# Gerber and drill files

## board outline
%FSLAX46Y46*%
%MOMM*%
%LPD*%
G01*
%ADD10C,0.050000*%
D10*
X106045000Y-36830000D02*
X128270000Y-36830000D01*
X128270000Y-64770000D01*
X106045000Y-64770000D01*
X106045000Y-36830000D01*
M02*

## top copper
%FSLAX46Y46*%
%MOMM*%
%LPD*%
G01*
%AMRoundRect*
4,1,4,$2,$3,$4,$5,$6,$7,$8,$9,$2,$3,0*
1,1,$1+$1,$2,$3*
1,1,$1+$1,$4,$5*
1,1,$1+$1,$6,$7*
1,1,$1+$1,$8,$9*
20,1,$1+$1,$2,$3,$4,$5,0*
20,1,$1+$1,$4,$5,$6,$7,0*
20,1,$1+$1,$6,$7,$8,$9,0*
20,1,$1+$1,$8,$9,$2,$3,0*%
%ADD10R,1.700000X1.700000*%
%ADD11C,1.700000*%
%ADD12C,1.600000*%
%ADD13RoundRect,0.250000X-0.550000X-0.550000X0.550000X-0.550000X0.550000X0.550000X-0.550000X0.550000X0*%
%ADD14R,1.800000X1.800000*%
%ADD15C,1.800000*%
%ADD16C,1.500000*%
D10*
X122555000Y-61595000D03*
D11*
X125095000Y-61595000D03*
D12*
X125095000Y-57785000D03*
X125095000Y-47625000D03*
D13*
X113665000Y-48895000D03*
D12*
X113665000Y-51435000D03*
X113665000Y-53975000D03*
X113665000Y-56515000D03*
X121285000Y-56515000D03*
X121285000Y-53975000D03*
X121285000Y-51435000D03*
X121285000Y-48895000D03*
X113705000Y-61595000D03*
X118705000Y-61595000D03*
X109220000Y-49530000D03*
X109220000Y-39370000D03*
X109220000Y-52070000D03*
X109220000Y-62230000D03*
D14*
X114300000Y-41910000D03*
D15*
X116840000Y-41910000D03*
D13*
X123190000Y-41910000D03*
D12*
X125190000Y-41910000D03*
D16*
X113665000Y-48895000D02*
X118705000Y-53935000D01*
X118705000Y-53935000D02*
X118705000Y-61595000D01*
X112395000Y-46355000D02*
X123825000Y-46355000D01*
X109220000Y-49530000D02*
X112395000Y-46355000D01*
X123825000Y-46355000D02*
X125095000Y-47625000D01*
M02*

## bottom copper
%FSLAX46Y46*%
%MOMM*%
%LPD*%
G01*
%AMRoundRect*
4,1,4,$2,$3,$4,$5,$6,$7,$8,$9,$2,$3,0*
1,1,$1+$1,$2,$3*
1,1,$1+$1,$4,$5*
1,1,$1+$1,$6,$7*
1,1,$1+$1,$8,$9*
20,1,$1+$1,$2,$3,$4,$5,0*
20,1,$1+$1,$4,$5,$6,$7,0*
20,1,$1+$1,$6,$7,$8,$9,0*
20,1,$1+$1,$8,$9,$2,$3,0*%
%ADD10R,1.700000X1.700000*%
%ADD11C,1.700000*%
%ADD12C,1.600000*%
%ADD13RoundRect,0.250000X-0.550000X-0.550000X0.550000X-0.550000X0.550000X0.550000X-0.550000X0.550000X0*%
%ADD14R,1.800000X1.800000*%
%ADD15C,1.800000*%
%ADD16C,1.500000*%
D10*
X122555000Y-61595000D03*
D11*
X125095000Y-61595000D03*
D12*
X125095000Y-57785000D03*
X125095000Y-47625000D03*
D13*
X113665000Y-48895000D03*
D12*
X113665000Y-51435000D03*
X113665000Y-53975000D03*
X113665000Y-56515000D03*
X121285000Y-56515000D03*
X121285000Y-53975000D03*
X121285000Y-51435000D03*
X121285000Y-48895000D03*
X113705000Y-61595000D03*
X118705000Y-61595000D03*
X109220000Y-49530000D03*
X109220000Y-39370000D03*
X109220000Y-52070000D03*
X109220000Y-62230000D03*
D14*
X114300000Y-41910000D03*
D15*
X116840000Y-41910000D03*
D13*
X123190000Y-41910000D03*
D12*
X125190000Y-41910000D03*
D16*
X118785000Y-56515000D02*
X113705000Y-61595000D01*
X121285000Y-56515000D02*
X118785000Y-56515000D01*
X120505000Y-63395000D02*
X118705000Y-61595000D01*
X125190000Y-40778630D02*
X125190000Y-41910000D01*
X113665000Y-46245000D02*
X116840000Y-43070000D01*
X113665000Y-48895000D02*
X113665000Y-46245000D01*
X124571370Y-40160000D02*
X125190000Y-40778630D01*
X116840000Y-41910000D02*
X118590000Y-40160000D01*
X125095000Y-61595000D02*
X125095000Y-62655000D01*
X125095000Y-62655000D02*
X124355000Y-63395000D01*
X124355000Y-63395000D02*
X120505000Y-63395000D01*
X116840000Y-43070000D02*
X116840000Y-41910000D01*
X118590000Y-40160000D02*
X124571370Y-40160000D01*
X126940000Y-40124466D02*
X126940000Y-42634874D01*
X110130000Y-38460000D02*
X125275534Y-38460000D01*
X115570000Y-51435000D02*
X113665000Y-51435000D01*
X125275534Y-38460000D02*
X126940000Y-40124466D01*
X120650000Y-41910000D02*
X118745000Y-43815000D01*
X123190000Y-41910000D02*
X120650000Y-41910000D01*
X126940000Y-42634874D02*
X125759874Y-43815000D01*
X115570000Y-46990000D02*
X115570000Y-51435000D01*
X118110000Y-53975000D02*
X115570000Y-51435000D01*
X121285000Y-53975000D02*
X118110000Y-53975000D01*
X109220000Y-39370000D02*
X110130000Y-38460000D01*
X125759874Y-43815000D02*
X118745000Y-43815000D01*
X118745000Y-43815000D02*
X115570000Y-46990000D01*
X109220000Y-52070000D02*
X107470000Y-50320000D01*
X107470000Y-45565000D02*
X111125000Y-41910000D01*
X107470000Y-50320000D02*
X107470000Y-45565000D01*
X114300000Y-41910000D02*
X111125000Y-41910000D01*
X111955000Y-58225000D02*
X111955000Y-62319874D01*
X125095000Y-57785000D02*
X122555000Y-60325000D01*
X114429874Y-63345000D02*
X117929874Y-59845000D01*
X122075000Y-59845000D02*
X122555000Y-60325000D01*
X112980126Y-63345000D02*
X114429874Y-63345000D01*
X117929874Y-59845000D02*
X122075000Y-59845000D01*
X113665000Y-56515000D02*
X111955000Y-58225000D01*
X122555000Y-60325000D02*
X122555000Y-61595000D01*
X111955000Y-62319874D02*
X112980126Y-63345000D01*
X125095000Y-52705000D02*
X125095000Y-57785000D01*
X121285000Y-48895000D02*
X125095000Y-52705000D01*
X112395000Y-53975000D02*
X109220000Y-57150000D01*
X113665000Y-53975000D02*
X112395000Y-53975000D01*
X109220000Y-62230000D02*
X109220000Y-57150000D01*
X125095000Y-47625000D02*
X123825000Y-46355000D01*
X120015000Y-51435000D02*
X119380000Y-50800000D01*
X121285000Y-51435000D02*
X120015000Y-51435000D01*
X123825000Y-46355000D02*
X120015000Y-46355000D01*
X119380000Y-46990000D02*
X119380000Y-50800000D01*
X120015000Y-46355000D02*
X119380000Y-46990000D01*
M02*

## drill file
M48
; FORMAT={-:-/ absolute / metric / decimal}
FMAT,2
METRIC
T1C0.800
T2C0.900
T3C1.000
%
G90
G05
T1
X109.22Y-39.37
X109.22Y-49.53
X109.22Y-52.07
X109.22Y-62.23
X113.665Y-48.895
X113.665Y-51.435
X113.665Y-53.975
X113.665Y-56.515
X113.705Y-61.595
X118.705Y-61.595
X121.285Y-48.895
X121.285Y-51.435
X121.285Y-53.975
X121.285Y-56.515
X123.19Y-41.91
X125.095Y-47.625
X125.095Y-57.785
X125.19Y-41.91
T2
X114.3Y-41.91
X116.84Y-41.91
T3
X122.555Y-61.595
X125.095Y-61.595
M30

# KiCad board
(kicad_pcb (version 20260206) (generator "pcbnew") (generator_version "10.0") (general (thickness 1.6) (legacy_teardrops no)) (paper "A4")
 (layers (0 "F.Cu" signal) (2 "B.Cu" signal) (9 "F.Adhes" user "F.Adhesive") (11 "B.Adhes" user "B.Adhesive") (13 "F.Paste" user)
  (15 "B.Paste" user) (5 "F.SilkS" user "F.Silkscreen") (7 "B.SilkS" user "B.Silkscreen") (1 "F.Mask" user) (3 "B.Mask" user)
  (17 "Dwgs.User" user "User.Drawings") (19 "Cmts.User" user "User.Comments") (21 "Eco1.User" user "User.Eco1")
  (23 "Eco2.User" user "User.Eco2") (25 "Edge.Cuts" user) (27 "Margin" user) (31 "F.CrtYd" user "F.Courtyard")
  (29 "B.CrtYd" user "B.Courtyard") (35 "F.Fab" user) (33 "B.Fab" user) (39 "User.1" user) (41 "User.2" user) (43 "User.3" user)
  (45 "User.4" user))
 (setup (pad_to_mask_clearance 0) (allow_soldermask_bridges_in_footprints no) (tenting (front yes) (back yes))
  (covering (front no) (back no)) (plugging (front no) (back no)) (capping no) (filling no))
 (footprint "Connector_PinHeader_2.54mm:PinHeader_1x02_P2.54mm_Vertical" (layer "F.Cu") (at 122.555 61.595 90)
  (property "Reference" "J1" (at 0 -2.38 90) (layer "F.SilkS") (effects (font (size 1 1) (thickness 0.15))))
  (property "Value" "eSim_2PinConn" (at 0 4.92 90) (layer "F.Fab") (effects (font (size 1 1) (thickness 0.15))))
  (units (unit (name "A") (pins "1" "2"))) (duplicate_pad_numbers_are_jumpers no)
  (pad "1" thru_hole rect (at 0 0 90) (size 1.7 1.7) (drill 1) (layers "*.Cu" "*.Mask") (remove_unused_layers no) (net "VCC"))
  (pad "2" thru_hole circle (at 0 2.54 90) (size 1.7 1.7) (drill 1) (layers "*.Cu" "*.Mask") (remove_unused_layers no) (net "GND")))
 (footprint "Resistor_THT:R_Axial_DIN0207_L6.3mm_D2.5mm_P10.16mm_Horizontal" (layer "F.Cu") (at 125.095 57.785 90)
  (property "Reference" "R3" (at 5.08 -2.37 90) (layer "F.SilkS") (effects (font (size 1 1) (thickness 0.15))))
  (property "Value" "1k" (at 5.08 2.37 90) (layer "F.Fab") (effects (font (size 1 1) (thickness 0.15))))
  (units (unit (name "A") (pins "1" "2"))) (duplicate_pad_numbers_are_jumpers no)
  (pad "1" thru_hole circle (at 0 0 90) (size 1.6 1.6) (drill 0.8) (layers "*.Cu" "*.Mask") (remove_unused_layers no) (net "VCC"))
  (pad "2" thru_hole circle (at 10.16 0 90) (size 1.6 1.6) (drill 0.8) (layers "*.Cu" "*.Mask") (remove_unused_layers no)
   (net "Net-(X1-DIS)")))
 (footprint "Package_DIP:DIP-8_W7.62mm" (layer "F.Cu") (at 113.665 48.895)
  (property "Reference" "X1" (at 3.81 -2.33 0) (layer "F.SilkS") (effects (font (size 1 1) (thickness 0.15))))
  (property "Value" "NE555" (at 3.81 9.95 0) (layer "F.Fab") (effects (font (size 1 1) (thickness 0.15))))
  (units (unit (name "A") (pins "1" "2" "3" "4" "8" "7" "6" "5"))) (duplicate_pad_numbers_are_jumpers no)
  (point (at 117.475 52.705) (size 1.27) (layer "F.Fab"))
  (pad "1" thru_hole roundrect (at 0 0) (size 1.6 1.6) (drill 0.8) (layers "*.Cu" "*.Mask") (remove_unused_layers no)
   (roundrect_rratio 0.15625) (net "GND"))
  (pad "2" thru_hole circle (at 0 2.54) (size 1.6 1.6) (drill 0.8) (layers "*.Cu" "*.Mask") (remove_unused_layers no) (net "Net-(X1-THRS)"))
  (pad "3" thru_hole circle (at 0 5.08) (size 1.6 1.6) (drill 0.8) (layers "*.Cu" "*.Mask") (remove_unused_layers no) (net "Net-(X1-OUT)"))
  (pad "4" thru_hole circle (at 0 7.62) (size 1.6 1.6) (drill 0.8) (layers "*.Cu" "*.Mask") (remove_unused_layers no) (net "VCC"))
  (pad "5" thru_hole circle (at 7.62 7.62) (size 1.6 1.6) (drill 0.8) (layers "*.Cu" "*.Mask") (remove_unused_layers no) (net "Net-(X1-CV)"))
  (pad "6" thru_hole circle (at 7.62 5.08) (size 1.6 1.6) (drill 0.8) (layers "*.Cu" "*.Mask") (remove_unused_layers no)
   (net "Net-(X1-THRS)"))
  (pad "7" thru_hole circle (at 7.62 2.54) (size 1.6 1.6) (drill 0.8) (layers "*.Cu" "*.Mask") (remove_unused_layers no)
   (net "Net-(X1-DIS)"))
  (pad "8" thru_hole circle (at 7.62 0) (size 1.6 1.6) (drill 0.8) (layers "*.Cu" "*.Mask") (remove_unused_layers no) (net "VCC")))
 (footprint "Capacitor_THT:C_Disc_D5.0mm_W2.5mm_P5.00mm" (layer "F.Cu") (at 113.705 61.595)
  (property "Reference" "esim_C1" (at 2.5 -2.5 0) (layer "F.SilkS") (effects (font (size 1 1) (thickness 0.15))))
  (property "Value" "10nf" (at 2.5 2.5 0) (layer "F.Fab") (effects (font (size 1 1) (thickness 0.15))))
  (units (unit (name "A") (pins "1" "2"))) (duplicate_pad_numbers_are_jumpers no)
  (pad "1" thru_hole circle (at 0 0) (size 1.6 1.6) (drill 0.8) (layers "*.Cu" "*.Mask") (remove_unused_layers no) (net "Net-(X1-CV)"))
  (pad "2" thru_hole circle (at 5 0) (size 1.6 1.6) (drill 0.8) (layers "*.Cu" "*.Mask") (remove_unused_layers no) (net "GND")))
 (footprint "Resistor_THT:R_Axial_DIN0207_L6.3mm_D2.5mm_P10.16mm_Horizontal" (layer "F.Cu") (at 109.22 49.53 90)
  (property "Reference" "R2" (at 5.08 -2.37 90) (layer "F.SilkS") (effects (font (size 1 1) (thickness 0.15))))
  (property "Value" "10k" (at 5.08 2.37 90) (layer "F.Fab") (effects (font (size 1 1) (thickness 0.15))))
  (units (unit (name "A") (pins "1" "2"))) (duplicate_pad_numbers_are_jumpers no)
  (pad "1" thru_hole circle (at 0 0 90) (size 1.6 1.6) (drill 0.8) (layers "*.Cu" "*.Mask") (remove_unused_layers no) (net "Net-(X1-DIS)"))
  (pad "2" thru_hole circle (at 10.16 0 90) (size 1.6 1.6) (drill 0.8) (layers "*.Cu" "*.Mask") (remove_unused_layers no)
   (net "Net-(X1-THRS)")))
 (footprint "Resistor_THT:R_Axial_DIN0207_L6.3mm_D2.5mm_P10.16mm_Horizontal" (layer "F.Cu") (at 109.22 52.07 -90)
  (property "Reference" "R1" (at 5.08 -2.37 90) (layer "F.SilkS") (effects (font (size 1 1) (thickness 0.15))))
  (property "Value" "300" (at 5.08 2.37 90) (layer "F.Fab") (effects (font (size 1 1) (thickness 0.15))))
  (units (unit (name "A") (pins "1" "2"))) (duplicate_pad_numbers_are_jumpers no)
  (pad "1" thru_hole circle (at 0 0 270) (size 1.6 1.6) (drill 0.8) (layers "*.Cu" "*.Mask") (remove_unused_layers no)
   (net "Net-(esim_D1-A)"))
  (pad "2" thru_hole circle (at 10.16 0 270) (size 1.6 1.6) (drill 0.8) (layers "*.Cu" "*.Mask") (remove_unused_layers no)
   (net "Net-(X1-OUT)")))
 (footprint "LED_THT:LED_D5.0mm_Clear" (layer "F.Cu") (at 114.3 41.91)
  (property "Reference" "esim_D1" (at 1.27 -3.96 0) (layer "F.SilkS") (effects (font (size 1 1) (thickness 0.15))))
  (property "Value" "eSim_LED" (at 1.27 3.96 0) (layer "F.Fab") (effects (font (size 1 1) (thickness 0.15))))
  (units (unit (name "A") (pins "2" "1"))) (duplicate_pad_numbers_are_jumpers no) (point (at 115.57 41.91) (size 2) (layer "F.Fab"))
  (pad "1" thru_hole rect (at 0 0) (size 1.8 1.8) (drill 0.9) (layers "*.Cu" "*.Mask") (remove_unused_layers no) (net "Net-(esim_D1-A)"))
  (pad "2" thru_hole circle (at 2.54 0) (size 1.8 1.8) (drill 0.9) (layers "*.Cu" "*.Mask") (remove_unused_layers no) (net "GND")))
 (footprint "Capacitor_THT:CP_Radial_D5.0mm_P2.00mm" (layer "F.Cu") (at 123.19 41.91)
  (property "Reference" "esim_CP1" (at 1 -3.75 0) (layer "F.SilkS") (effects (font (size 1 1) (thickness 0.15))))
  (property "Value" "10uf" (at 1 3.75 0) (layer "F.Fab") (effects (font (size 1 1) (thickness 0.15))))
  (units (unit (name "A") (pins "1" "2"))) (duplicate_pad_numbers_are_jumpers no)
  (pad "1" thru_hole roundrect (at 0 0) (size 1.6 1.6) (drill 0.8) (layers "*.Cu" "*.Mask") (remove_unused_layers no)
   (roundrect_rratio 0.15625) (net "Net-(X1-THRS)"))
  (pad "2" thru_hole circle (at 2 0) (size 1.6 1.6) (drill 0.8) (layers "*.Cu" "*.Mask") (remove_unused_layers no) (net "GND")))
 (gr_rect (start 106.045 36.83) (end 128.27 64.77) (stroke (width 0.05) (type default)) (fill no) (layer "Edge.Cuts"))
 (segment (start 118.785 56.515) (end 113.705 61.595) (width 1.5) (layer "B.Cu") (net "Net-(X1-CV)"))
 (segment (start 121.285 56.515) (end 118.785 56.515) (width 1.5) (layer "B.Cu") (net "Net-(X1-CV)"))
 (segment (start 113.665 48.895) (end 118.705 53.935) (width 1.5) (layer "F.Cu") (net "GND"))
 (segment (start 118.705 53.935) (end 118.705 61.595) (width 1.5) (layer "F.Cu") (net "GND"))
 (segment (start 120.505 63.395) (end 118.705 61.595) (width 1.5) (layer "B.Cu") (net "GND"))
 (segment (start 125.19 40.77863) (end 125.19 41.91) (width 1.5) (layer "B.Cu") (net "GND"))
 (segment (start 113.665 46.245) (end 116.84 43.07) (width 1.5) (layer "B.Cu") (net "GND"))
 (segment (start 113.665 48.895) (end 113.665 46.245) (width 1.5) (layer "B.Cu") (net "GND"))
 (segment (start 124.57137 40.16) (end 125.19 40.77863) (width 1.5) (layer "B.Cu") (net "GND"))
 (segment (start 116.84 41.91) (end 118.59 40.16) (width 1.5) (layer "B.Cu") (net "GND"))
 (segment (start 125.095 61.595) (end 125.095 62.655) (width 1.5) (layer "B.Cu") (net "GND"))
 (segment (start 125.095 62.655) (end 124.355 63.395) (width 1.5) (layer "B.Cu") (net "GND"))
 (segment (start 124.355 63.395) (end 120.505 63.395) (width 1.5) (layer "B.Cu") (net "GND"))
 (segment (start 116.84 43.07) (end 116.84 41.91) (width 1.5) (layer "B.Cu") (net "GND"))
 (segment (start 118.59 40.16) (end 124.57137 40.16) (width 1.5) (layer "B.Cu") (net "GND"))
 (segment (start 126.94 40.124466) (end 126.94 42.634874) (width 1.5) (layer "B.Cu") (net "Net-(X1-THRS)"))
 (segment (start 110.13 38.46) (end 125.275534 38.46) (width 1.5) (layer "B.Cu") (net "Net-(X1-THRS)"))
 (segment (start 115.57 51.435) (end 113.665 51.435) (width 1.5) (layer "B.Cu") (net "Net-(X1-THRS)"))
 (segment (start 125.275534 38.46) (end 126.94 40.124466) (width 1.5) (layer "B.Cu") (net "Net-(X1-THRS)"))
 (segment (start 120.65 41.91) (end 118.745 43.815) (width 1.5) (layer "B.Cu") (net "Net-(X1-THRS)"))
 (segment (start 123.19 41.91) (end 120.65 41.91) (width 1.5) (layer "B.Cu") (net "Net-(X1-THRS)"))
 (segment (start 126.94 42.634874) (end 125.759874 43.815) (width 1.5) (layer "B.Cu") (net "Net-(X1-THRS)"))
 (segment (start 115.57 46.99) (end 115.57 51.435) (width 1.5) (layer "B.Cu") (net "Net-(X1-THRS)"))
 (segment (start 118.11 53.975) (end 115.57 51.435) (width 1.5) (layer "B.Cu") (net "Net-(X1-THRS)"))
 (segment (start 121.285 53.975) (end 118.11 53.975) (width 1.5) (layer "B.Cu") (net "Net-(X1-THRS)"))
 (segment (start 109.22 39.37) (end 110.13 38.46) (width 1.5) (layer "B.Cu") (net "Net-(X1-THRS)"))
 (segment (start 125.759874 43.815) (end 118.745 43.815) (width 1.5) (layer "B.Cu") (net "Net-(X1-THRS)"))
 (segment (start 118.745 43.815) (end 115.57 46.99) (width 1.5) (layer "B.Cu") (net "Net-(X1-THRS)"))
 (segment (start 109.22 52.07) (end 107.47 50.32) (width 1.5) (layer "B.Cu") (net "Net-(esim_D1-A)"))
 (segment (start 107.47 45.565) (end 111.125 41.91) (width 1.5) (layer "B.Cu") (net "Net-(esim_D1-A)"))
 (segment (start 107.47 50.32) (end 107.47 45.565) (width 1.5) (layer "B.Cu") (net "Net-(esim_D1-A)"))
 (segment (start 114.3 41.91) (end 111.125 41.91) (width 1.5) (layer "B.Cu") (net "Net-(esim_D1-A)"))
 (segment (start 111.955 58.225) (end 111.955 62.319874) (width 1.5) (layer "B.Cu") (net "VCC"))
 (segment (start 125.095 57.785) (end 122.555 60.325) (width 1.5) (layer "B.Cu") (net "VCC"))
 (segment (start 114.429874 63.345) (end 117.929874 59.845) (width 1.5) (layer "B.Cu") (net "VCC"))
 (segment (start 122.075 59.845) (end 122.555 60.325) (width 1.5) (layer "B.Cu") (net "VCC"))
 (segment (start 112.980126 63.345) (end 114.429874 63.345) (width 1.5) (layer "B.Cu") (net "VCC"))
 (segment (start 117.929874 59.845) (end 122.075 59.845) (width 1.5) (layer "B.Cu") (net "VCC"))
 (segment (start 113.665 56.515) (end 111.955 58.225) (width 1.5) (layer "B.Cu") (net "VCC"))
 (segment (start 122.555 60.325) (end 122.555 61.595) (width 1.5) (layer "B.Cu") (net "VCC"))
 (segment (start 111.955 62.319874) (end 112.980126 63.345) (width 1.5) (layer "B.Cu") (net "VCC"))
 (segment (start 125.095 52.705) (end 125.095 57.785) (width 1.5) (layer "B.Cu") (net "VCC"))
 (segment (start 121.285 48.895) (end 125.095 52.705) (width 1.5) (layer "B.Cu") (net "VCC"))
 (segment (start 112.395 53.975) (end 109.22 57.15) (width 1.5) (layer "B.Cu") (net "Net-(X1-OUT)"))
 (segment (start 113.665 53.975) (end 112.395 53.975) (width 1.5) (layer "B.Cu") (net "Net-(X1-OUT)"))
 (segment (start 109.22 62.23) (end 109.22 57.15) (width 1.5) (layer "B.Cu") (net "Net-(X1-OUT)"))
 (segment (start 112.395 46.355) (end 123.825 46.355) (width 1.5) (layer "F.Cu") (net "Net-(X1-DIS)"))
 (segment (start 109.22 49.53) (end 112.395 46.355) (width 1.5) (layer "F.Cu") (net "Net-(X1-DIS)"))
 (segment (start 123.825 46.355) (end 125.095 47.625) (width 1.5) (layer "F.Cu") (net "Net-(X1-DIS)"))
 (segment (start 125.095 47.625) (end 123.825 46.355) (width 1.5) (layer "B.Cu") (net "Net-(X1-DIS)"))
 (segment (start 120.015 51.435) (end 119.38 50.8) (width 1.5) (layer "B.Cu") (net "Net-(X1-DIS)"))
 (segment (start 121.285 51.435) (end 120.015 51.435) (width 1.5) (layer "B.Cu") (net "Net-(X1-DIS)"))
 (segment (start 123.825 46.355) (end 120.015 46.355) (width 1.5) (layer "B.Cu") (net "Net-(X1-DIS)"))
 (segment (start 119.38 46.99) (end 119.38 50.8) (width 1.5) (layer "B.Cu") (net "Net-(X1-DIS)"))
 (segment (start 120.015 46.355) (end 119.38 46.99) (width 1.5) (layer "B.Cu") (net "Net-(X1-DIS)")))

